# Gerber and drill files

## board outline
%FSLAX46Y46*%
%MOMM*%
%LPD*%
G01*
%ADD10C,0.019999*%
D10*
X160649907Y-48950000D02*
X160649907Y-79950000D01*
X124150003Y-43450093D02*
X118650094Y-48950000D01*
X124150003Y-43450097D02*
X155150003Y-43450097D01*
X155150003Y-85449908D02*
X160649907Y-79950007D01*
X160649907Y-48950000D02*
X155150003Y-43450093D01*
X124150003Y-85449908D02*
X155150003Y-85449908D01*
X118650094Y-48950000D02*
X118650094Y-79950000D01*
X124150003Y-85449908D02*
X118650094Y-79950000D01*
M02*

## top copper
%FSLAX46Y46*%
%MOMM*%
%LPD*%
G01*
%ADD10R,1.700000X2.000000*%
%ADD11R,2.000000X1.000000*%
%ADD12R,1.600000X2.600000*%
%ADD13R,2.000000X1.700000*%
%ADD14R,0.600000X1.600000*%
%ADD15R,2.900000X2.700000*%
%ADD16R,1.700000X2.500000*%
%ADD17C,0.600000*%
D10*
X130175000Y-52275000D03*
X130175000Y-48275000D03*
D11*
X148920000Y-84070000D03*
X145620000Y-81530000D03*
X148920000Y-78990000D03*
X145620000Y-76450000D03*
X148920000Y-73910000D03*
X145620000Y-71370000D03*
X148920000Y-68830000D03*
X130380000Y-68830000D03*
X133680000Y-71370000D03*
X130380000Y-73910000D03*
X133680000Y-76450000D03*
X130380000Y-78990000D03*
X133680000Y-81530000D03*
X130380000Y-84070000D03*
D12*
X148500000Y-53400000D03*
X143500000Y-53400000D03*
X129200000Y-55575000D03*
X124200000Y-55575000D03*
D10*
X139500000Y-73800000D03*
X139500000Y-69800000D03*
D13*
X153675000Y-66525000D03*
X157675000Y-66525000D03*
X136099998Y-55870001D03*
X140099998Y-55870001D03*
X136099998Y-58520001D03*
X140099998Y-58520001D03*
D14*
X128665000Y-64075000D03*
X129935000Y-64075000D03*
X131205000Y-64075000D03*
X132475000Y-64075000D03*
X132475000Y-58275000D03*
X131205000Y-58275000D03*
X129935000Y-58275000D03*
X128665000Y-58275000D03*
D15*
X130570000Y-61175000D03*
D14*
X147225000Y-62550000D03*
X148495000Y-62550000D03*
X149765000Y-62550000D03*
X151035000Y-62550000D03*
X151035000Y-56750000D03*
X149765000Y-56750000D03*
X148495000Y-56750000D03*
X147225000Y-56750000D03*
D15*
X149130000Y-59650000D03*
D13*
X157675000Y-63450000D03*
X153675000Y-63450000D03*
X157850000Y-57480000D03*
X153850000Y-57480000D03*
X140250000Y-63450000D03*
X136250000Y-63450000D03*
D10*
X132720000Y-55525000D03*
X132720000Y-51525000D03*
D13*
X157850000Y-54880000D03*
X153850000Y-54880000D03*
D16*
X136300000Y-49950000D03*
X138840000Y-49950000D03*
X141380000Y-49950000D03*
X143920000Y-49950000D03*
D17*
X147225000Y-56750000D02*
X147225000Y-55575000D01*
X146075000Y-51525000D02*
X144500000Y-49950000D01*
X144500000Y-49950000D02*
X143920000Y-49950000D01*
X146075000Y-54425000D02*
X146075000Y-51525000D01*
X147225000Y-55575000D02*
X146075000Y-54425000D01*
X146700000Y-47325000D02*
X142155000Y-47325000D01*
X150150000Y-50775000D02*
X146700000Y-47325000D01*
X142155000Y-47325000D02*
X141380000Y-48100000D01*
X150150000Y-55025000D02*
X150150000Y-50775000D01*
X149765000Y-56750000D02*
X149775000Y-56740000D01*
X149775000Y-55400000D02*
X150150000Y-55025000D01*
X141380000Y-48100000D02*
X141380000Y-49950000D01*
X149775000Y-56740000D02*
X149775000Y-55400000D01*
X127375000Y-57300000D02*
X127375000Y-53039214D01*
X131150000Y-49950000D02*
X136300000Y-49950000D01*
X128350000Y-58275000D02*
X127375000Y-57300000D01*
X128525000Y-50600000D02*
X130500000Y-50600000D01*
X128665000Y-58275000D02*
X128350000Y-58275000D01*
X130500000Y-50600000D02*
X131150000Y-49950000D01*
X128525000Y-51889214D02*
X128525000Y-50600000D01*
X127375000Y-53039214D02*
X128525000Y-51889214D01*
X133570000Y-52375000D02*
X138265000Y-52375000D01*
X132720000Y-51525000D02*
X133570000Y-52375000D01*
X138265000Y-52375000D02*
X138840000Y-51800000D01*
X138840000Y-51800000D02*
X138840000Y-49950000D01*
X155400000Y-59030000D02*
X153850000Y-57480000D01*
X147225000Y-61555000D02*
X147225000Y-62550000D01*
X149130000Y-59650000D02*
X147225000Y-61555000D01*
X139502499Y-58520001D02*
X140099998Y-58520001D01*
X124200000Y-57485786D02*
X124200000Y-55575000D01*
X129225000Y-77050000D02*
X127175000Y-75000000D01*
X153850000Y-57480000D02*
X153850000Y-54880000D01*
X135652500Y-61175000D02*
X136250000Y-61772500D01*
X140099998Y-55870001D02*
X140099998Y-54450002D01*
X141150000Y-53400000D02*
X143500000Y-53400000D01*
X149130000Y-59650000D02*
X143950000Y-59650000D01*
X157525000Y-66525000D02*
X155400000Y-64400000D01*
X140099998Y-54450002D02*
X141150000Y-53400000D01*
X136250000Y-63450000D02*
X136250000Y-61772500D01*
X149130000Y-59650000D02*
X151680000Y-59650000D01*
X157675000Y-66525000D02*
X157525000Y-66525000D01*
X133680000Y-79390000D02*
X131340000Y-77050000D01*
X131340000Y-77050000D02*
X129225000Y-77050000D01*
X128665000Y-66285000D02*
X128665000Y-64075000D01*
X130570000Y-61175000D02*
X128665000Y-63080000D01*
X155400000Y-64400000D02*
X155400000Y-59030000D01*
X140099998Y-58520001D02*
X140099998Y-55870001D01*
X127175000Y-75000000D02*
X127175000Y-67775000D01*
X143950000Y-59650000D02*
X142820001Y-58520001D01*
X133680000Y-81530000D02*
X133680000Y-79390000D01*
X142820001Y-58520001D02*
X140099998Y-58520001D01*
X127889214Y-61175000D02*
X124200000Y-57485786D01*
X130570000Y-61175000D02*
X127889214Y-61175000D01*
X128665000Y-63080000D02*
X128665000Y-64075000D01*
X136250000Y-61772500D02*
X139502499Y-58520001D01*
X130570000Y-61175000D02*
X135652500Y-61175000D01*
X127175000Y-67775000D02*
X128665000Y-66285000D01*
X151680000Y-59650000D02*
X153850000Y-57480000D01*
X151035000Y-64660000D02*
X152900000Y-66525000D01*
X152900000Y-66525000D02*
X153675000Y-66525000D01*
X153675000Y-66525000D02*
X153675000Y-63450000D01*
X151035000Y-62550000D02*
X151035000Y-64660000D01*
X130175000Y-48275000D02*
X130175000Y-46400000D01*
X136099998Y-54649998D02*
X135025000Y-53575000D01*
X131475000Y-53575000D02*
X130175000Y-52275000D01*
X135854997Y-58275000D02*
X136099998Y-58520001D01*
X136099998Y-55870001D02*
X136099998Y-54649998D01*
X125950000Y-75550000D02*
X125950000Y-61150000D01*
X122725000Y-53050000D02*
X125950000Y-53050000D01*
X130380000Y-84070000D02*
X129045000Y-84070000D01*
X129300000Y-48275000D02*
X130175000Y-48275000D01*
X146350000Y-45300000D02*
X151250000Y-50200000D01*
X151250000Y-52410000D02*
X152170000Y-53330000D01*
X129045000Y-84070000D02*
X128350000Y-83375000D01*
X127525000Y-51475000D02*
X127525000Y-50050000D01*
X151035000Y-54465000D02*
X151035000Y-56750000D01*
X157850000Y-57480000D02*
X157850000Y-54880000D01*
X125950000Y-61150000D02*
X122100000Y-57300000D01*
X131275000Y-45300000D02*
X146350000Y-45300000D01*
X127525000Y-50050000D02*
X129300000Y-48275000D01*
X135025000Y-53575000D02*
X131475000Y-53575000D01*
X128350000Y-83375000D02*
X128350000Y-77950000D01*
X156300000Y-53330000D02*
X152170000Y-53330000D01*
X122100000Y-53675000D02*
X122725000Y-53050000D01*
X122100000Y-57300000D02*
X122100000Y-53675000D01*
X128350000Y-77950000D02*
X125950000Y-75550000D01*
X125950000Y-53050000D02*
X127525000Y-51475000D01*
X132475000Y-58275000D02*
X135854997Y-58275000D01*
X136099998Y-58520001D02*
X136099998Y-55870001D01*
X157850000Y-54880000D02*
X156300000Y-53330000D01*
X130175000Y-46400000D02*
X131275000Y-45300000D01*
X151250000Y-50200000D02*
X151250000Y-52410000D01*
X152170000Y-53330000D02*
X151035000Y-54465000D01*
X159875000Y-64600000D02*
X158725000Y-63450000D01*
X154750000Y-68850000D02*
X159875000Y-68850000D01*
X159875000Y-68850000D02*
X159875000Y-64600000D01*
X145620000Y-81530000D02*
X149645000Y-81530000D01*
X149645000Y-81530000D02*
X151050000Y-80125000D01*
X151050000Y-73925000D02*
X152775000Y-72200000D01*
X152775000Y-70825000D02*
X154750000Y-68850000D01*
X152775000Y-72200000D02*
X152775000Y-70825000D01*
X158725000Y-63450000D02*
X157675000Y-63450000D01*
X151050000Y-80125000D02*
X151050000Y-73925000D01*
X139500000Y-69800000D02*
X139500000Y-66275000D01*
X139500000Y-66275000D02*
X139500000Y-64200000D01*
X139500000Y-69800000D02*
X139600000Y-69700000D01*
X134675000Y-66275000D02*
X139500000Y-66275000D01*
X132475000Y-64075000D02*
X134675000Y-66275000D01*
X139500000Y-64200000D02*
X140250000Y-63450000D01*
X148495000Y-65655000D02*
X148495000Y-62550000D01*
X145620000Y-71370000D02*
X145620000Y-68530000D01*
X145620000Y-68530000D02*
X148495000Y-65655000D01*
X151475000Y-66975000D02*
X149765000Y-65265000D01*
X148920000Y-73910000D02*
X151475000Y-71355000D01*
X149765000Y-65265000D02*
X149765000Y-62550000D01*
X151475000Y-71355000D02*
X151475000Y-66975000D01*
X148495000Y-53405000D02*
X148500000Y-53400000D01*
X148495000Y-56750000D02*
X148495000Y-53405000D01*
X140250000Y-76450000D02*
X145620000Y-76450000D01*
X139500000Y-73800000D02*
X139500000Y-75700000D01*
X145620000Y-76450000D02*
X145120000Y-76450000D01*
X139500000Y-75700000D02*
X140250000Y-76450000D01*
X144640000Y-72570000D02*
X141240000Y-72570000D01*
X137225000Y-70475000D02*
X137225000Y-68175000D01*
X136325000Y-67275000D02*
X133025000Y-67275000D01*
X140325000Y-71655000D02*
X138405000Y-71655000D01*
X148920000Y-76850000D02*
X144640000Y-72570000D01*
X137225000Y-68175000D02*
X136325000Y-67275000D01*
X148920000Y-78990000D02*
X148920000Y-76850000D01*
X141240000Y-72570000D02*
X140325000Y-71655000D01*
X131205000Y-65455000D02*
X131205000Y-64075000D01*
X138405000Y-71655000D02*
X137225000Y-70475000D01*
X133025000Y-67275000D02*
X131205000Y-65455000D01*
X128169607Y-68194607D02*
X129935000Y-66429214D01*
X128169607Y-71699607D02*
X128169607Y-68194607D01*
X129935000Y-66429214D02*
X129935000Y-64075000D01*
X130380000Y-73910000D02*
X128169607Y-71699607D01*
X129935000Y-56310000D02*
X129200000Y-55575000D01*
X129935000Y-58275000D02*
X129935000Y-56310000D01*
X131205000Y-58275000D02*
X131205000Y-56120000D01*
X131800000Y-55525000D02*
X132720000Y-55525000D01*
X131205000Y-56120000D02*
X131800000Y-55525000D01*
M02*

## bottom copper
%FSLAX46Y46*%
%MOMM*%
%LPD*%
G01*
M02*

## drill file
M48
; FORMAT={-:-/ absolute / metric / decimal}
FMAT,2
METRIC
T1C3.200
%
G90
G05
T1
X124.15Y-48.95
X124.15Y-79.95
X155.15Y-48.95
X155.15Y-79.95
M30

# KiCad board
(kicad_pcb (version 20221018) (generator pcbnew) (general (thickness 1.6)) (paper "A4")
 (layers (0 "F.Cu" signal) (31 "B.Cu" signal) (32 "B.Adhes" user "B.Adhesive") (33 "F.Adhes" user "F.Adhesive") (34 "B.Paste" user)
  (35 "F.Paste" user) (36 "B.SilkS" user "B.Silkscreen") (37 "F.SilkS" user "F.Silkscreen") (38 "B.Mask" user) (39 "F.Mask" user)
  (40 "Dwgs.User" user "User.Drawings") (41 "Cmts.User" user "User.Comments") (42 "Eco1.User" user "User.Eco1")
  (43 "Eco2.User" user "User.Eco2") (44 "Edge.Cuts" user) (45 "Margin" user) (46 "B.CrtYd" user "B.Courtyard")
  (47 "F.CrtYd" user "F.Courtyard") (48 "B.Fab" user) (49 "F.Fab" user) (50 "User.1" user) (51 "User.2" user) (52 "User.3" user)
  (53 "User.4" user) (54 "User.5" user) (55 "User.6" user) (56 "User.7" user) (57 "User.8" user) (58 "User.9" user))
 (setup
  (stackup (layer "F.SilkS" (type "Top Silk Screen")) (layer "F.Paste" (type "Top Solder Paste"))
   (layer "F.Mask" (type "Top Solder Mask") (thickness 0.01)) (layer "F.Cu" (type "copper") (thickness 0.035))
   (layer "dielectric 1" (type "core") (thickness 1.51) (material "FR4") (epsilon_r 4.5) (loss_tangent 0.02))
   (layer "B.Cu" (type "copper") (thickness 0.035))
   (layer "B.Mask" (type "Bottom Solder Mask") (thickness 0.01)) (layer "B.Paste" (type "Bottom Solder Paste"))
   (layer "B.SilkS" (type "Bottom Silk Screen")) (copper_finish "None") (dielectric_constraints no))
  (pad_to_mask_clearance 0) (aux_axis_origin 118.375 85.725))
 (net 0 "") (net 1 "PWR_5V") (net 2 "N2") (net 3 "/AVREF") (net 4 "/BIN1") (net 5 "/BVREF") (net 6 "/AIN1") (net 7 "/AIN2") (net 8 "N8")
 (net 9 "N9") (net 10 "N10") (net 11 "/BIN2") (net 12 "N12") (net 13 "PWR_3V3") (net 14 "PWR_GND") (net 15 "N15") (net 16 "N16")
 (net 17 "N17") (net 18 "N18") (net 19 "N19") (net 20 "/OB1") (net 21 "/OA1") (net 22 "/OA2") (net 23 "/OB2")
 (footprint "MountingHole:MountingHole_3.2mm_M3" (layer "F.Cu") (at 124.15 48.95)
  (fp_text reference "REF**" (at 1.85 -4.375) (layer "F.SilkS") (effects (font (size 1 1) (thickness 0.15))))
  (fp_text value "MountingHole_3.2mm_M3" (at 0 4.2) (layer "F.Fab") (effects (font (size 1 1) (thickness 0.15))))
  (pad "" np_thru_hole circle (at 0 0) (size 3.2 3.2) (drill 3.2) (layers "*.Cu" "*.Mask")))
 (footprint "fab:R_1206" (layer "F.Cu") (at 130.175 50.275 90)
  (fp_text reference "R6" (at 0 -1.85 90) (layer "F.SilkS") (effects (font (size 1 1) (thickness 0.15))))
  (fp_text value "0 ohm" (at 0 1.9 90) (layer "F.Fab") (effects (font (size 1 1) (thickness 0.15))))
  (pad "1" smd rect (at -2 0 90) (size 2 1.7) (layers "F.Cu" "F.Paste" "F.Mask") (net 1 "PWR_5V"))
  (pad "2" smd rect (at 2 0 90) (size 2 1.7) (layers "F.Cu" "F.Paste" "F.Mask") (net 1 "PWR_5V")))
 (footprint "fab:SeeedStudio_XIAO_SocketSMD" (layer "F.Cu") (at 139.65 76.45 180)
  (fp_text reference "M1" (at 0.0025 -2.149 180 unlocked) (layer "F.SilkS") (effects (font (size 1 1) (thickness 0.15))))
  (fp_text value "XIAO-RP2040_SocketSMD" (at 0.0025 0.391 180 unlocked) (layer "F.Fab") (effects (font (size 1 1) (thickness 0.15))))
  (pad "1" smd rect (at -9.27 -7.62 180) (size 2 1) (layers "F.Cu" "F.Paste" "F.Mask") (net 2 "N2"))
  (pad "2" smd rect (at -5.97 -5.08 180) (size 2 1) (layers "F.Cu" "F.Paste" "F.Mask") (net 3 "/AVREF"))
  (pad "3" smd rect (at -9.27 -2.54 180) (size 2 1) (layers "F.Cu" "F.Paste" "F.Mask") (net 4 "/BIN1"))
  (pad "4" smd rect (at -5.97 0 180) (size 2 1) (layers "F.Cu" "F.Paste" "F.Mask") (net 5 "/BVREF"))
  (pad "5" smd rect (at -9.27 2.54 180) (size 2 1) (layers "F.Cu" "F.Paste" "F.Mask") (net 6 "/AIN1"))
  (pad "6" smd rect (at -5.97 5.08 180) (size 2 1) (layers "F.Cu" "F.Paste" "F.Mask") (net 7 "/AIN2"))
  (pad "7" smd rect (at -9.27 7.62 180) (size 2 1) (layers "F.Cu" "F.Paste" "F.Mask") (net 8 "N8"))
  (pad "8" smd rect (at 9.27 7.62 180) (size 2 1) (layers "F.Cu" "F.Paste" "F.Mask") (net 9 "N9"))
  (pad "9" smd rect (at 5.97 5.08 180) (size 2 1) (layers "F.Cu" "F.Paste" "F.Mask") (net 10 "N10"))
  (pad "10" smd rect (at 9.27 2.54 180) (size 2 1) (layers "F.Cu" "F.Paste" "F.Mask") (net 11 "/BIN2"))
  (pad "11" smd rect (at 5.97 0 180) (size 2 1) (layers "F.Cu" "F.Paste" "F.Mask") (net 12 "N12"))
  (pad "12" smd rect (at 9.27 -2.54 180) (size 2 1) (layers "F.Cu" "F.Paste" "F.Mask") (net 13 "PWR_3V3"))
  (pad "13" smd rect (at 5.97 -5.08 180) (size 2 1) (layers "F.Cu" "F.Paste" "F.Mask") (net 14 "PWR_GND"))
  (pad "14" smd rect (at 9.27 -7.62 180) (size 2 1) (layers "F.Cu" "F.Paste" "F.Mask") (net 1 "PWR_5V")))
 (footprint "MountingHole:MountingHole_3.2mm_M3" (layer "F.Cu") (at 155.15 79.95)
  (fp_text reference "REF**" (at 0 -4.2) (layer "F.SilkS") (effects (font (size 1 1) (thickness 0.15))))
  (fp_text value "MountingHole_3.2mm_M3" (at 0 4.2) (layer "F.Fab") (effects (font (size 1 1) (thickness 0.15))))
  (pad "" np_thru_hole circle (at 0 0) (size 3.2 3.2) (drill 3.2) (layers "*.Cu" "*.Mask")))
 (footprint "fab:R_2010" (layer "F.Cu") (at 146 53.4 180)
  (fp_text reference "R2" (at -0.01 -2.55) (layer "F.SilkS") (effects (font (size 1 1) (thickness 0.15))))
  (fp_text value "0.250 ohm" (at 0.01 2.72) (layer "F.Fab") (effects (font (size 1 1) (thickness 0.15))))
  (pad "1" smd rect (at -2.5 0 180) (size 1.6 2.6) (layers "F.Cu" "F.Paste" "F.Mask") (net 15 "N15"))
  (pad "2" smd rect (at 2.5 0 180) (size 1.6 2.6) (layers "F.Cu" "F.Paste" "F.Mask") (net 14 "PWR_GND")))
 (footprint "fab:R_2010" (layer "F.Cu") (at 126.7 55.575 180)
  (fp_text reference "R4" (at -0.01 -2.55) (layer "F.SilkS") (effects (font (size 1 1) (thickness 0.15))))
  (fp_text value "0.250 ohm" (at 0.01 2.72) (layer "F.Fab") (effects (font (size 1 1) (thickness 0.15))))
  (pad "1" smd rect (at -2.5 0 180) (size 1.6 2.6) (layers "F.Cu" "F.Paste" "F.Mask") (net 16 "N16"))
  (pad "2" smd rect (at 2.5 0 180) (size 1.6 2.6) (layers "F.Cu" "F.Paste" "F.Mask") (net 14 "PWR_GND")))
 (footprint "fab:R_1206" (layer "F.Cu") (at 139.5 71.8 90)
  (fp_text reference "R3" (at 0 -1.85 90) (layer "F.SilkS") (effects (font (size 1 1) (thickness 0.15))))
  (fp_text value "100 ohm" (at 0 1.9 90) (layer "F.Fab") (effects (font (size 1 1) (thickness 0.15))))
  (pad "1" smd rect (at -2 0 90) (size 2 1.7) (layers "F.Cu" "F.Paste" "F.Mask") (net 5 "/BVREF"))
  (pad "2" smd rect (at 2 0 90) (size 2 1.7) (layers "F.Cu" "F.Paste" "F.Mask") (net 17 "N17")))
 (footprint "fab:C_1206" (layer "F.Cu") (at 155.675 66.525)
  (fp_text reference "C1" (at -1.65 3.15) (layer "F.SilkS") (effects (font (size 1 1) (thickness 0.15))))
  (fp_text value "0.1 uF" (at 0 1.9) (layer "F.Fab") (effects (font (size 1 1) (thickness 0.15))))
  (pad "1" smd rect (at -2 0) (size 2 1.7) (layers "F.Cu" "F.Paste" "F.Mask") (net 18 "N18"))
  (pad "2" smd rect (at 2 0) (size 2 1.7) (layers "F.Cu" "F.Paste" "F.Mask") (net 14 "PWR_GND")))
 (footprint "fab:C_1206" (layer "F.Cu") (at 138.099998 55.870001)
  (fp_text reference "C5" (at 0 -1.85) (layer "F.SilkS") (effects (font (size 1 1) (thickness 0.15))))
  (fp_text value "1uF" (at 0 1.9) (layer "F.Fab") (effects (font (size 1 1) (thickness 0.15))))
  (pad "1" smd rect (at -2 0) (size 2 1.7) (layers "F.Cu" "F.Paste" "F.Mask") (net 1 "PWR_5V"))
  (pad "2" smd rect (at 2 0) (size 2 1.7) (layers "F.Cu" "F.Paste" "F.Mask") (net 14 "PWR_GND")))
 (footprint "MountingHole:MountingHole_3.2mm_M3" (layer "F.Cu") (at 155.15 48.95)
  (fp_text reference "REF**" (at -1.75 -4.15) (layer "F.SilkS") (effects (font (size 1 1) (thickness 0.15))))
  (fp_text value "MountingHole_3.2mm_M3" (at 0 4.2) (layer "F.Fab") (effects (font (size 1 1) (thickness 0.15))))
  (pad "" np_thru_hole circle (at 0 0) (size 3.2 3.2) (drill 3.2) (layers "*.Cu" "*.Mask")))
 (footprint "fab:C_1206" (layer "F.Cu") (at 138.099998 58.520001)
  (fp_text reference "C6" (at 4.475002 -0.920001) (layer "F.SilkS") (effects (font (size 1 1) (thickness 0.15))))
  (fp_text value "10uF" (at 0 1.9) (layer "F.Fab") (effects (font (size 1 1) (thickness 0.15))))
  (pad "1" smd rect (at -2 0) (size 2 1.7) (layers "F.Cu" "F.Paste" "F.Mask") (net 1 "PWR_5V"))
  (pad "2" smd rect (at 2 0) (size 2 1.7) (layers "F.Cu" "F.Paste" "F.Mask") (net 14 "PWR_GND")))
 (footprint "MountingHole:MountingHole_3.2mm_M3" (layer "F.Cu") (at 124.15 79.95)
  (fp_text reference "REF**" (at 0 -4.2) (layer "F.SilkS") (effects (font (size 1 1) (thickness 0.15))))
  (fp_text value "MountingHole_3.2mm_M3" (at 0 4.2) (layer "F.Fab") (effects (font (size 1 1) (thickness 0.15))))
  (pad "" np_thru_hole circle (at 0 0) (size 3.2 3.2) (drill 3.2) (layers "*.Cu" "*.Mask")))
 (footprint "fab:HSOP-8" (layer "F.Cu") (at 130.57 61.175 90)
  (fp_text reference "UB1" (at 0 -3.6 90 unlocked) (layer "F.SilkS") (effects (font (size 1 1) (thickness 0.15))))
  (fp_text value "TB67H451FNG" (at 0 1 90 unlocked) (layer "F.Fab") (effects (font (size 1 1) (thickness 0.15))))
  (pad "1" smd rect (at -2.9 -1.905 90) (size 1.6 0.6) (layers "F.Cu" "F.Paste" "F.Mask") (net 14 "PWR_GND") (thermal_bridge_angle 45))
  (pad "2" smd rect (at -2.9 -0.635 90) (size 1.6 0.6) (layers "F.Cu" "F.Paste" "F.Mask") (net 11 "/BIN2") (thermal_bridge_angle 45))
  (pad "3" smd rect (at -2.9 0.635 90) (size 1.6 0.6) (layers "F.Cu" "F.Paste" "F.Mask") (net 4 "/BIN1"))
  (pad "4" smd rect (at -2.9 1.905 90) (size 1.6 0.6) (layers "F.Cu" "F.Paste" "F.Mask") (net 17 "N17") (thermal_bridge_angle 45))
  (pad "5" smd rect (at 2.9 1.905 90) (size 1.6 0.6) (layers "F.Cu" "F.Paste" "F.Mask") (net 1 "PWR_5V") (thermal_bridge_angle 45))
  (pad "6" smd rect (at 2.9 0.635 90) (size 1.6 0.6) (layers "F.Cu" "F.Paste" "F.Mask") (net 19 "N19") (thermal_bridge_angle 45))
  (pad "7" smd rect (at 2.9 -0.635 90) (size 1.6 0.6) (layers "F.Cu" "F.Paste" "F.Mask") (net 16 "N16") (thermal_bridge_angle 45))
  (pad "8" smd rect (at 2.9 -1.905 90) (size 1.6 0.6) (layers "F.Cu" "F.Paste" "F.Mask") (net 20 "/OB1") (thermal_bridge_angle 45))
  (pad "9" smd rect (at 0 0 90) (size 2.7 2.9) (layers "F.Cu" "F.Paste" "F.Mask") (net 14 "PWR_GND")))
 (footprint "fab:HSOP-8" (layer "F.Cu") (at 149.13 59.65 90)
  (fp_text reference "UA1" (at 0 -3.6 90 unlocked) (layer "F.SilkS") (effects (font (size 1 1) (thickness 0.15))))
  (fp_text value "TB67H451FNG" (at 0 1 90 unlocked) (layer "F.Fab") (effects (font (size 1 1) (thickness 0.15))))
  (pad "1" smd rect (at -2.9 -1.905 90) (size 1.6 0.6) (layers "F.Cu" "F.Paste" "F.Mask") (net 14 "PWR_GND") (thermal_bridge_angle 45))
  (pad "2" smd rect (at -2.9 -0.635 90) (size 1.6 0.6) (layers "F.Cu" "F.Paste" "F.Mask") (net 7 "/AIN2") (thermal_bridge_angle 45))
  (pad "3" smd rect (at -2.9 0.635 90) (size 1.6 0.6) (layers "F.Cu" "F.Paste" "F.Mask") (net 6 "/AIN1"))
  (pad "4" smd rect (at -2.9 1.905 90) (size 1.6 0.6) (layers "F.Cu" "F.Paste" "F.Mask") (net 18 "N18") (thermal_bridge_angle 45))
  (pad "5" smd rect (at 2.9 1.905 90) (size 1.6 0.6) (layers "F.Cu" "F.Paste" "F.Mask") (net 1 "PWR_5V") (thermal_bridge_angle 45))
  (pad "6" smd rect (at 2.9 0.635 90) (size 1.6 0.6) (layers "F.Cu" "F.Paste" "F.Mask") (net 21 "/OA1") (thermal_bridge_angle 45))
  (pad "7" smd rect (at 2.9 -0.635 90) (size 1.6 0.6) (layers "F.Cu" "F.Paste" "F.Mask") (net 15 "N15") (thermal_bridge_angle 45))
  (pad "8" smd rect (at 2.9 -1.905 90) (size 1.6 0.6) (layers "F.Cu" "F.Paste" "F.Mask") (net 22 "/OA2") (thermal_bridge_angle 45))
  (pad "9" smd rect (at 0 0 90) (size 2.7 2.9) (layers "F.Cu" "F.Paste" "F.Mask") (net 14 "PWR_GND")))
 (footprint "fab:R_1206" (layer "F.Cu") (at 155.675 63.45 180)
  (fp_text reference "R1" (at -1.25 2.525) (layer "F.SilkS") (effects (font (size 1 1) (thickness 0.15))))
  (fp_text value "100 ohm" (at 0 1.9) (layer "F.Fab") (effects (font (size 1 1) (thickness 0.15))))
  (pad "1" smd rect (at -2 0 180) (size 2 1.7) (layers "F.Cu" "F.Paste" "F.Mask") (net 3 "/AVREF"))
  (pad "2" smd rect (at 2 0 180) (size 2 1.7) (layers "F.Cu" "F.Paste" "F.Mask") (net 18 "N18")))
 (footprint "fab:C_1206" (layer "F.Cu") (at 155.85 57.48 180)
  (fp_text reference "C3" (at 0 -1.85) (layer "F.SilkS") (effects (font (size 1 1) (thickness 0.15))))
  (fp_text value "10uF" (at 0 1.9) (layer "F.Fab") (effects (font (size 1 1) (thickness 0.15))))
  (pad "1" smd rect (at -2 0 180) (size 2 1.7) (layers "F.Cu" "F.Paste" "F.Mask") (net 1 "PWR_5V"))
  (pad "2" smd rect (at 2 0 180) (size 2 1.7) (layers "F.Cu" "F.Paste" "F.Mask") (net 14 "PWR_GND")))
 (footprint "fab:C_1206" (layer "F.Cu") (at 138.25 63.45 180)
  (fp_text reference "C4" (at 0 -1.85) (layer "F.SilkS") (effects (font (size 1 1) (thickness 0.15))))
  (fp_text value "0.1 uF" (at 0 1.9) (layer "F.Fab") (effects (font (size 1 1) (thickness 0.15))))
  (pad "1" smd rect (at -2 0 180) (size 2 1.7) (layers "F.Cu" "F.Paste" "F.Mask") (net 17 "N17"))
  (pad "2" smd rect (at 2 0 180) (size 2 1.7) (layers "F.Cu" "F.Paste" "F.Mask") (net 14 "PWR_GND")))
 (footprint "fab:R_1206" (layer "F.Cu") (at 132.72 53.525 90)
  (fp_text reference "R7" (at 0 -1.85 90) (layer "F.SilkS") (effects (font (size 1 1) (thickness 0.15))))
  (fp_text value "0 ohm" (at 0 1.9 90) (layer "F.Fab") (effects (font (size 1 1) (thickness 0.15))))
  (pad "1" smd rect (at -2 0 90) (size 2 1.7) (layers "F.Cu" "F.Paste" "F.Mask") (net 19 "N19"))
  (pad "2" smd rect (at 2 0 90) (size 2 1.7) (layers "F.Cu" "F.Paste" "F.Mask") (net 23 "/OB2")))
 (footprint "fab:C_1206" (layer "F.Cu") (at 155.85 54.88 180)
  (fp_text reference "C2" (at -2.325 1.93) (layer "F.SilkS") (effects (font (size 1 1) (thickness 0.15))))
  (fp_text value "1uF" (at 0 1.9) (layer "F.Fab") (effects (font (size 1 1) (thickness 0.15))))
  (pad "1" smd rect (at -2 0 180) (size 2 1.7) (layers "F.Cu" "F.Paste" "F.Mask") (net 1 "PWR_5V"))
  (pad "2" smd rect (at 2 0 180) (size 2 1.7) (layers "F.Cu" "F.Paste" "F.Mask") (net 14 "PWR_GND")))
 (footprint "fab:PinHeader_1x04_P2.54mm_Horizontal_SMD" (layer "F.Cu") (at 136.3 49.95 90)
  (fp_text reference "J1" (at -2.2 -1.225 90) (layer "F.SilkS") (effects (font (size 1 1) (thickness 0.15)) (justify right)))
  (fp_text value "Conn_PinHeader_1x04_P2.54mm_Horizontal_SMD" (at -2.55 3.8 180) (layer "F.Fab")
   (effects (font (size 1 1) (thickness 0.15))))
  (pad "1" smd rect (at 0 0 90) (size 2.5 1.7) (layers "F.Cu" "F.Paste" "F.Mask") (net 20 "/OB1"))
  (pad "2" smd rect (at 0 2.54 90) (size 2.5 1.7) (layers "F.Cu" "F.Paste" "F.Mask") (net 23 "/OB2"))
  (pad "3" smd rect (at 0 5.08 90) (size 2.5 1.7) (layers "F.Cu" "F.Paste" "F.Mask") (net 21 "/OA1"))
  (pad "4" smd rect (at 0 7.62 90) (size 2.5 1.7) (layers "F.Cu" "F.Paste" "F.Mask") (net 22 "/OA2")))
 (gr_line (start 160.649907 48.95) (end 160.649907 79.95) (stroke (width 0.019999) (type solid)) (layer "Edge.Cuts"))
 (gr_line (start 124.150003 43.450093) (end 118.650094 48.95) (stroke (width 0.019999) (type solid)) (layer "Edge.Cuts"))
 (gr_line (start 124.150003 43.450097) (end 155.150003 43.450097) (stroke (width 0.019999) (type solid)) (layer "Edge.Cuts"))
 (gr_line (start 155.150003 85.449908) (end 160.649907 79.950007) (stroke (width 0.019999) (type solid)) (layer "Edge.Cuts"))
 (gr_line (start 160.649907 48.95) (end 155.150003 43.450093) (stroke (width 0.019999) (type solid)) (layer "Edge.Cuts"))
 (gr_line (start 124.150003 85.449908) (end 155.150003 85.449908) (stroke (width 0.019999) (type solid)) (layer "Edge.Cuts"))
 (gr_line (start 118.650094 48.95) (end 118.650094 79.95) (stroke (width 0.019999) (type solid)) (layer "Edge.Cuts"))
 (gr_line (start 124.150003 85.449908) (end 118.650094 79.95) (stroke (width 0.019999) (type solid)) (layer "Edge.Cuts"))
 (segment (start 147.225 56.75) (end 147.225 55.575) (width 0.6) (layer "F.Cu") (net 22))
 (segment (start 146.075 51.525) (end 144.5 49.95) (width 0.6) (layer "F.Cu") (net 22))
 (segment (start 144.5 49.95) (end 143.92 49.95) (width 0.6) (layer "F.Cu") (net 22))
 (segment (start 146.075 54.425) (end 146.075 51.525) (width 0.6) (layer "F.Cu") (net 22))
 (segment (start 147.225 55.575) (end 146.075 54.425) (width 0.6) (layer "F.Cu") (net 22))
 (segment (start 146.7 47.325) (end 142.155 47.325) (width 0.6) (layer "F.Cu") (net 21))
 (segment (start 150.15 50.775) (end 146.7 47.325) (width 0.6) (layer "F.Cu") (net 21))
 (segment (start 142.155 47.325) (end 141.38 48.1) (width 0.6) (layer "F.Cu") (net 21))
 (segment (start 150.15 55.025) (end 150.15 50.775) (width 0.6) (layer "F.Cu") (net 21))
 (segment (start 149.765 56.75) (end 149.775 56.74) (width 0.6) (layer "F.Cu") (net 21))
 (segment (start 149.775 55.4) (end 150.15 55.025) (width 0.6) (layer "F.Cu") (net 21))
 (segment (start 141.38 48.1) (end 141.38 49.95) (width 0.6) (layer "F.Cu") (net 21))
 (segment (start 149.775 56.74) (end 149.775 55.4) (width 0.6) (layer "F.Cu") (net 21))
 (segment (start 127.375 57.3) (end 127.375 53.039214) (width 0.6) (layer "F.Cu") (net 20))
 (segment (start 131.15 49.95) (end 136.3 49.95) (width 0.6) (layer "F.Cu") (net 20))
 (segment (start 128.35 58.275) (end 127.375 57.3) (width 0.6) (layer "F.Cu") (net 20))
 (segment (start 128.525 50.6) (end 130.5 50.6) (width 0.6) (layer "F.Cu") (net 20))
 (segment (start 128.665 58.275) (end 128.35 58.275) (width 0.6) (layer "F.Cu") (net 20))
 (segment (start 130.5 50.6) (end 131.15 49.95) (width 0.6) (layer "F.Cu") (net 20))
 (segment (start 128.525 51.889214) (end 128.525 50.6) (width 0.6) (layer "F.Cu") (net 20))
 (segment (start 127.375 53.039214) (end 128.525 51.889214) (width 0.6) (layer "F.Cu") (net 20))
 (segment (start 133.57 52.375) (end 138.265 52.375) (width 0.6) (layer "F.Cu") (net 23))
 (segment (start 132.72 51.525) (end 133.57 52.375) (width 0.6) (layer "F.Cu") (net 23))
 (segment (start 138.265 52.375) (end 138.84 51.8) (width 0.6) (layer "F.Cu") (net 23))
 (segment (start 138.84 51.8) (end 138.84 49.95) (width 0.6) (layer "F.Cu") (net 23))
 (segment (start 155.4 59.03) (end 153.85 57.48) (width 0.6) (layer "F.Cu") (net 14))
 (segment (start 147.225 61.555) (end 147.225 62.55) (width 0.6) (layer "F.Cu") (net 14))
 (segment (start 149.13 59.65) (end 147.225 61.555) (width 0.6) (layer "F.Cu") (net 14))
 (segment (start 139.502499 58.520001) (end 140.099998 58.520001) (width 0.6) (layer "F.Cu") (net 14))
 (segment (start 124.2 57.485786) (end 124.2 55.575) (width 0.6) (layer "F.Cu") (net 14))
 (segment (start 129.225 77.05) (end 127.175 75) (width 0.6) (layer "F.Cu") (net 14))
 (segment (start 153.85 57.48) (end 153.85 54.88) (width 0.6) (layer "F.Cu") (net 14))
 (segment (start 135.6525 61.175) (end 136.25 61.7725) (width 0.6) (layer "F.Cu") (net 14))
 (segment (start 140.099998 55.870001) (end 140.099998 54.450002) (width 0.6) (layer "F.Cu") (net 14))
 (segment (start 141.15 53.4) (end 143.5 53.4) (width 0.6) (layer "F.Cu") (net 14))
 (segment (start 149.13 59.65) (end 143.95 59.65) (width 0.6) (layer "F.Cu") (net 14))
 (segment (start 157.525 66.525) (end 155.4 64.4) (width 0.6) (layer "F.Cu") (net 14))
 (segment (start 140.099998 54.450002) (end 141.15 53.4) (width 0.6) (layer "F.Cu") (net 14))
 (segment (start 136.25 63.45) (end 136.25 61.7725) (width 0.6) (layer "F.Cu") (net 14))
 (segment (start 149.13 59.65) (end 151.68 59.65) (width 0.6) (layer "F.Cu") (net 14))
 (segment (start 157.675 66.525) (end 157.525 66.525) (width 0.6) (layer "F.Cu") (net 14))
 (segment (start 133.68 79.39) (end 131.34 77.05) (width 0.6) (layer "F.Cu") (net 14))
 (segment (start 131.34 77.05) (end 129.225 77.05) (width 0.6) (layer "F.Cu") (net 14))
 (segment (start 128.665 66.285) (end 128.665 64.075) (width 0.6) (layer "F.Cu") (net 14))
 (segment (start 130.57 61.175) (end 128.665 63.08) (width 0.6) (layer "F.Cu") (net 14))
 (segment (start 155.4 64.4) (end 155.4 59.03) (width 0.6) (layer "F.Cu") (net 14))
 (segment (start 140.099998 58.520001) (end 140.099998 55.870001) (width 0.6) (layer "F.Cu") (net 14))
 (segment (start 127.175 75) (end 127.175 67.775) (width 0.6) (layer "F.Cu") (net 14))
 (segment (start 143.95 59.65) (end 142.820001 58.520001) (width 0.6) (layer "F.Cu") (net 14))
 (segment (start 133.68 81.53) (end 133.68 79.39) (width 0.6) (layer "F.Cu") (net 14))
 (segment (start 142.820001 58.520001) (end 140.099998 58.520001) (width 0.6) (layer "F.Cu") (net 14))
 (segment (start 127.889214 61.175) (end 124.2 57.485786) (width 0.6) (layer "F.Cu") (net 14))
 (segment (start 130.57 61.175) (end 127.889214 61.175) (width 0.6) (layer "F.Cu") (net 14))
 (segment (start 128.665 63.08) (end 128.665 64.075) (width 0.6) (layer "F.Cu") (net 14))
 (segment (start 136.25 61.7725) (end 139.502499 58.520001) (width 0.6) (layer "F.Cu") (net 14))
 (segment (start 130.57 61.175) (end 135.6525 61.175) (width 0.6) (layer "F.Cu") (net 14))
 (segment (start 127.175 67.775) (end 128.665 66.285) (width 0.6) (layer "F.Cu") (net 14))
 (segment (start 151.68 59.65) (end 153.85 57.48) (width 0.6) (layer "F.Cu") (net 14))
 (segment (start 151.035 64.66) (end 152.9 66.525) (width 0.6) (layer "F.Cu") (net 18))
 (segment (start 152.9 66.525) (end 153.675 66.525) (width 0.6) (layer "F.Cu") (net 18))
 (segment (start 153.675 66.525) (end 153.675 63.45) (width 0.6) (layer "F.Cu") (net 18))
 (segment (start 151.035 62.55) (end 151.035 64.66) (width 0.6) (layer "F.Cu") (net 18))
 (segment (start 130.175 48.275) (end 130.175 46.4) (width 0.6) (layer "F.Cu") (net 1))
 (segment (start 136.099998 54.649998) (end 135.025 53.575) (width 0.6) (layer "F.Cu") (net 1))
 (segment (start 131.475 53.575) (end 130.175 52.275) (width 0.6) (layer "F.Cu") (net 1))
 (segment (start 135.854997 58.275) (end 136.099998 58.520001) (width 0.6) (layer "F.Cu") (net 1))
 (segment (start 136.099998 55.870001) (end 136.099998 54.649998) (width 0.6) (layer "F.Cu") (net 1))
 (segment (start 125.95 75.55) (end 125.95 61.15) (width 0.6) (layer "F.Cu") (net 1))
 (segment (start 122.725 53.05) (end 125.95 53.05) (width 0.6) (layer "F.Cu") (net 1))
 (segment (start 130.38 84.07) (end 129.045 84.07) (width 0.6) (layer "F.Cu") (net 1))
 (segment (start 129.3 48.275) (end 130.175 48.275) (width 0.6) (layer "F.Cu") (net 1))
 (segment (start 146.35 45.3) (end 151.25 50.2) (width 0.6) (layer "F.Cu") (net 1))
 (segment (start 151.25 52.41) (end 152.17 53.33) (width 0.6) (layer "F.Cu") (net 1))
 (segment (start 129.045 84.07) (end 128.35 83.375) (width 0.6) (layer "F.Cu") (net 1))
 (segment (start 127.525 51.475) (end 127.525 50.05) (width 0.6) (layer "F.Cu") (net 1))
 (segment (start 151.035 54.465) (end 151.035 56.75) (width 0.6) (layer "F.Cu") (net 1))
 (segment (start 157.85 57.48) (end 157.85 54.88) (width 0.6) (layer "F.Cu") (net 1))
 (segment (start 125.95 61.15) (end 122.1 57.3) (width 0.6) (layer "F.Cu") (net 1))
 (segment (start 131.275 45.3) (end 146.35 45.3) (width 0.6) (layer "F.Cu") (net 1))
 (segment (start 127.525 50.05) (end 129.3 48.275) (width 0.6) (layer "F.Cu") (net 1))
 (segment (start 135.025 53.575) (end 131.475 53.575) (width 0.6) (layer "F.Cu") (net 1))
 (segment (start 128.35 83.375) (end 128.35 77.95) (width 0.6) (layer "F.Cu") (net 1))
 (segment (start 156.3 53.33) (end 152.17 53.33) (width 0.6) (layer "F.Cu") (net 1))
 (segment (start 122.1 53.675) (end 122.725 53.05) (width 0.6) (layer "F.Cu") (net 1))
 (segment (start 122.1 57.3) (end 122.1 53.675) (width 0.6) (layer "F.Cu") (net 1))
 (segment (start 128.35 77.95) (end 125.95 75.55) (width 0.6) (layer "F.Cu") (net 1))
 (segment (start 125.95 53.05) (end 127.525 51.475) (width 0.6) (layer "F.Cu") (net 1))
 (segment (start 132.475 58.275) (end 135.854997 58.275) (width 0.6) (layer "F.Cu") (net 1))
 (segment (start 136.099998 58.520001) (end 136.099998 55.870001) (width 0.6) (layer "F.Cu") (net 1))
 (segment (start 157.85 54.88) (end 156.3 53.33) (width 0.6) (layer "F.Cu") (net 1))
 (segment (start 130.175 46.4) (end 131.275 45.3) (width 0.6) (layer "F.Cu") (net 1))
 (segment (start 151.25 50.2) (end 151.25 52.41) (width 0.6) (layer "F.Cu") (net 1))
 (segment (start 152.17 53.33) (end 151.035 54.465) (width 0.6) (layer "F.Cu") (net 1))
 (segment (start 159.875 64.6) (end 158.725 63.45) (width 0.6) (layer "F.Cu") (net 3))
 (segment (start 154.75 68.85) (end 159.875 68.85) (width 0.6) (layer "F.Cu") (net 3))
 (segment (start 159.875 68.85) (end 159.875 64.6) (width 0.6) (layer "F.Cu") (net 3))
 (segment (start 145.62 81.53) (end 149.645 81.53) (width 0.6) (layer "F.Cu") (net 3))
 (segment (start 149.645 81.53) (end 151.05 80.125) (width 0.6) (layer "F.Cu") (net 3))
 (segment (start 151.05 73.925) (end 152.775 72.2) (width 0.6) (layer "F.Cu") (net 3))
 (segment (start 152.775 70.825) (end 154.75 68.85) (width 0.6) (layer "F.Cu") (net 3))
 (segment (start 152.775 72.2) (end 152.775 70.825) (width 0.6) (layer "F.Cu") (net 3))
 (segment (start 158.725 63.45) (end 157.675 63.45) (width 0.6) (layer "F.Cu") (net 3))
 (segment (start 151.05 80.125) (end 151.05 73.925) (width 0.6) (layer "F.Cu") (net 3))
 (segment (start 139.5 69.8) (end 139.5 66.275) (width 0.6) (layer "F.Cu") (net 17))
 (segment (start 139.5 66.275) (end 139.5 64.2) (width 0.6) (layer "F.Cu") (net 17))
 (segment (start 139.5 69.8) (end 139.6 69.7) (width 0.6) (layer "F.Cu") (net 17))
 (segment (start 134.675 66.275) (end 139.5 66.275) (width 0.6) (layer "F.Cu") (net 17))
 (segment (start 132.475 64.075) (end 134.675 66.275) (width 0.6) (layer "F.Cu") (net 17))
 (segment (start 139.5 64.2) (end 140.25 63.45) (width 0.6) (layer "F.Cu") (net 17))
 (segment (start 148.495 65.655) (end 148.495 62.55) (width 0.6) (layer "F.Cu") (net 7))
 (segment (start 145.62 71.37) (end 145.62 68.53) (width 0.6) (layer "F.Cu") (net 7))
 (segment (start 145.62 68.53) (end 148.495 65.655) (width 0.6) (layer "F.Cu") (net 7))
 (segment (start 151.475 66.975) (end 149.765 65.265) (width 0.6) (layer "F.Cu") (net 6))
 (segment (start 148.92 73.91) (end 151.475 71.355) (width 0.6) (layer "F.Cu") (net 6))
 (segment (start 149.765 65.265) (end 149.765 62.55) (width 0.6) (layer "F.Cu") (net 6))
 (segment (start 151.475 71.355) (end 151.475 66.975) (width 0.6) (layer "F.Cu") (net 6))
 (segment (start 148.495 53.405) (end 148.5 53.4) (width 0.6) (layer "F.Cu") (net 15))
 (segment (start 148.495 56.75) (end 148.495 53.405) (width 0.6) (layer "F.Cu") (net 15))
 (segment (start 140.25 76.45) (end 145.62 76.45) (width 0.6) (layer "F.Cu") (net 5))
 (segment (start 139.5 73.8) (end 139.5 75.7) (width 0.6) (layer "F.Cu") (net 5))
 (segment (start 145.62 76.45) (end 145.12 76.45) (width 0.6) (layer "F.Cu") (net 5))
 (segment (start 139.5 75.7) (end 140.25 76.45) (width 0.6) (layer "F.Cu") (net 5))
 (segment (start 144.64 72.57) (end 141.24 72.57) (width 0.6) (layer "F.Cu") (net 4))
 (segment (start 137.225 70.475) (end 137.225 68.175) (width 0.6) (layer "F.Cu") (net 4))
 (segment (start 136.325 67.275) (end 133.025 67.275) (width 0.6) (layer "F.Cu") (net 4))
 (segment (start 140.325 71.655) (end 138.405 71.655) (width 0.6) (layer "F.Cu") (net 4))
 (segment (start 148.92 76.85) (end 144.64 72.57) (width 0.6) (layer "F.Cu") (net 4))
 (segment (start 137.225 68.175) (end 136.325 67.275) (width 0.6) (layer "F.Cu") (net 4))
 (segment (start 148.92 78.99) (end 148.92 76.85) (width 0.6) (layer "F.Cu") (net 4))
 (segment (start 141.24 72.57) (end 140.325 71.655) (width 0.6) (layer "F.Cu") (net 4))
 (segment (start 131.205 65.455) (end 131.205 64.075) (width 0.6) (layer "F.Cu") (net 4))
 (segment (start 138.405 71.655) (end 137.225 70.475) (width 0.6) (layer "F.Cu") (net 4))
 (segment (start 133.025 67.275) (end 131.205 65.455) (width 0.6) (layer "F.Cu") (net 4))
 (segment (start 128.169607 68.194607) (end 129.935 66.429214) (width 0.6) (layer "F.Cu") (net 11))
 (segment (start 128.169607 71.699607) (end 128.169607 68.194607) (width 0.6) (layer "F.Cu") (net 11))
 (segment (start 129.935 66.429214) (end 129.935 64.075) (width 0.6) (layer "F.Cu") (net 11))
 (segment (start 130.38 73.91) (end 128.169607 71.699607) (width 0.6) (layer "F.Cu") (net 11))
 (segment (start 129.935 56.31) (end 129.2 55.575) (width 0.6) (layer "F.Cu") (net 16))
 (segment (start 129.935 58.275) (end 129.935 56.31) (width 0.6) (layer "F.Cu") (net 16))
 (segment (start 131.205 58.275) (end 131.205 56.12) (width 0.6) (layer "F.Cu") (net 19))
 (segment (start 131.8 55.525) (end 132.72 55.525) (width 0.6) (layer "F.Cu") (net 19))
 (segment (start 131.205 56.12) (end 131.8 55.525) (width 0.6) (layer "F.Cu") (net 19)))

